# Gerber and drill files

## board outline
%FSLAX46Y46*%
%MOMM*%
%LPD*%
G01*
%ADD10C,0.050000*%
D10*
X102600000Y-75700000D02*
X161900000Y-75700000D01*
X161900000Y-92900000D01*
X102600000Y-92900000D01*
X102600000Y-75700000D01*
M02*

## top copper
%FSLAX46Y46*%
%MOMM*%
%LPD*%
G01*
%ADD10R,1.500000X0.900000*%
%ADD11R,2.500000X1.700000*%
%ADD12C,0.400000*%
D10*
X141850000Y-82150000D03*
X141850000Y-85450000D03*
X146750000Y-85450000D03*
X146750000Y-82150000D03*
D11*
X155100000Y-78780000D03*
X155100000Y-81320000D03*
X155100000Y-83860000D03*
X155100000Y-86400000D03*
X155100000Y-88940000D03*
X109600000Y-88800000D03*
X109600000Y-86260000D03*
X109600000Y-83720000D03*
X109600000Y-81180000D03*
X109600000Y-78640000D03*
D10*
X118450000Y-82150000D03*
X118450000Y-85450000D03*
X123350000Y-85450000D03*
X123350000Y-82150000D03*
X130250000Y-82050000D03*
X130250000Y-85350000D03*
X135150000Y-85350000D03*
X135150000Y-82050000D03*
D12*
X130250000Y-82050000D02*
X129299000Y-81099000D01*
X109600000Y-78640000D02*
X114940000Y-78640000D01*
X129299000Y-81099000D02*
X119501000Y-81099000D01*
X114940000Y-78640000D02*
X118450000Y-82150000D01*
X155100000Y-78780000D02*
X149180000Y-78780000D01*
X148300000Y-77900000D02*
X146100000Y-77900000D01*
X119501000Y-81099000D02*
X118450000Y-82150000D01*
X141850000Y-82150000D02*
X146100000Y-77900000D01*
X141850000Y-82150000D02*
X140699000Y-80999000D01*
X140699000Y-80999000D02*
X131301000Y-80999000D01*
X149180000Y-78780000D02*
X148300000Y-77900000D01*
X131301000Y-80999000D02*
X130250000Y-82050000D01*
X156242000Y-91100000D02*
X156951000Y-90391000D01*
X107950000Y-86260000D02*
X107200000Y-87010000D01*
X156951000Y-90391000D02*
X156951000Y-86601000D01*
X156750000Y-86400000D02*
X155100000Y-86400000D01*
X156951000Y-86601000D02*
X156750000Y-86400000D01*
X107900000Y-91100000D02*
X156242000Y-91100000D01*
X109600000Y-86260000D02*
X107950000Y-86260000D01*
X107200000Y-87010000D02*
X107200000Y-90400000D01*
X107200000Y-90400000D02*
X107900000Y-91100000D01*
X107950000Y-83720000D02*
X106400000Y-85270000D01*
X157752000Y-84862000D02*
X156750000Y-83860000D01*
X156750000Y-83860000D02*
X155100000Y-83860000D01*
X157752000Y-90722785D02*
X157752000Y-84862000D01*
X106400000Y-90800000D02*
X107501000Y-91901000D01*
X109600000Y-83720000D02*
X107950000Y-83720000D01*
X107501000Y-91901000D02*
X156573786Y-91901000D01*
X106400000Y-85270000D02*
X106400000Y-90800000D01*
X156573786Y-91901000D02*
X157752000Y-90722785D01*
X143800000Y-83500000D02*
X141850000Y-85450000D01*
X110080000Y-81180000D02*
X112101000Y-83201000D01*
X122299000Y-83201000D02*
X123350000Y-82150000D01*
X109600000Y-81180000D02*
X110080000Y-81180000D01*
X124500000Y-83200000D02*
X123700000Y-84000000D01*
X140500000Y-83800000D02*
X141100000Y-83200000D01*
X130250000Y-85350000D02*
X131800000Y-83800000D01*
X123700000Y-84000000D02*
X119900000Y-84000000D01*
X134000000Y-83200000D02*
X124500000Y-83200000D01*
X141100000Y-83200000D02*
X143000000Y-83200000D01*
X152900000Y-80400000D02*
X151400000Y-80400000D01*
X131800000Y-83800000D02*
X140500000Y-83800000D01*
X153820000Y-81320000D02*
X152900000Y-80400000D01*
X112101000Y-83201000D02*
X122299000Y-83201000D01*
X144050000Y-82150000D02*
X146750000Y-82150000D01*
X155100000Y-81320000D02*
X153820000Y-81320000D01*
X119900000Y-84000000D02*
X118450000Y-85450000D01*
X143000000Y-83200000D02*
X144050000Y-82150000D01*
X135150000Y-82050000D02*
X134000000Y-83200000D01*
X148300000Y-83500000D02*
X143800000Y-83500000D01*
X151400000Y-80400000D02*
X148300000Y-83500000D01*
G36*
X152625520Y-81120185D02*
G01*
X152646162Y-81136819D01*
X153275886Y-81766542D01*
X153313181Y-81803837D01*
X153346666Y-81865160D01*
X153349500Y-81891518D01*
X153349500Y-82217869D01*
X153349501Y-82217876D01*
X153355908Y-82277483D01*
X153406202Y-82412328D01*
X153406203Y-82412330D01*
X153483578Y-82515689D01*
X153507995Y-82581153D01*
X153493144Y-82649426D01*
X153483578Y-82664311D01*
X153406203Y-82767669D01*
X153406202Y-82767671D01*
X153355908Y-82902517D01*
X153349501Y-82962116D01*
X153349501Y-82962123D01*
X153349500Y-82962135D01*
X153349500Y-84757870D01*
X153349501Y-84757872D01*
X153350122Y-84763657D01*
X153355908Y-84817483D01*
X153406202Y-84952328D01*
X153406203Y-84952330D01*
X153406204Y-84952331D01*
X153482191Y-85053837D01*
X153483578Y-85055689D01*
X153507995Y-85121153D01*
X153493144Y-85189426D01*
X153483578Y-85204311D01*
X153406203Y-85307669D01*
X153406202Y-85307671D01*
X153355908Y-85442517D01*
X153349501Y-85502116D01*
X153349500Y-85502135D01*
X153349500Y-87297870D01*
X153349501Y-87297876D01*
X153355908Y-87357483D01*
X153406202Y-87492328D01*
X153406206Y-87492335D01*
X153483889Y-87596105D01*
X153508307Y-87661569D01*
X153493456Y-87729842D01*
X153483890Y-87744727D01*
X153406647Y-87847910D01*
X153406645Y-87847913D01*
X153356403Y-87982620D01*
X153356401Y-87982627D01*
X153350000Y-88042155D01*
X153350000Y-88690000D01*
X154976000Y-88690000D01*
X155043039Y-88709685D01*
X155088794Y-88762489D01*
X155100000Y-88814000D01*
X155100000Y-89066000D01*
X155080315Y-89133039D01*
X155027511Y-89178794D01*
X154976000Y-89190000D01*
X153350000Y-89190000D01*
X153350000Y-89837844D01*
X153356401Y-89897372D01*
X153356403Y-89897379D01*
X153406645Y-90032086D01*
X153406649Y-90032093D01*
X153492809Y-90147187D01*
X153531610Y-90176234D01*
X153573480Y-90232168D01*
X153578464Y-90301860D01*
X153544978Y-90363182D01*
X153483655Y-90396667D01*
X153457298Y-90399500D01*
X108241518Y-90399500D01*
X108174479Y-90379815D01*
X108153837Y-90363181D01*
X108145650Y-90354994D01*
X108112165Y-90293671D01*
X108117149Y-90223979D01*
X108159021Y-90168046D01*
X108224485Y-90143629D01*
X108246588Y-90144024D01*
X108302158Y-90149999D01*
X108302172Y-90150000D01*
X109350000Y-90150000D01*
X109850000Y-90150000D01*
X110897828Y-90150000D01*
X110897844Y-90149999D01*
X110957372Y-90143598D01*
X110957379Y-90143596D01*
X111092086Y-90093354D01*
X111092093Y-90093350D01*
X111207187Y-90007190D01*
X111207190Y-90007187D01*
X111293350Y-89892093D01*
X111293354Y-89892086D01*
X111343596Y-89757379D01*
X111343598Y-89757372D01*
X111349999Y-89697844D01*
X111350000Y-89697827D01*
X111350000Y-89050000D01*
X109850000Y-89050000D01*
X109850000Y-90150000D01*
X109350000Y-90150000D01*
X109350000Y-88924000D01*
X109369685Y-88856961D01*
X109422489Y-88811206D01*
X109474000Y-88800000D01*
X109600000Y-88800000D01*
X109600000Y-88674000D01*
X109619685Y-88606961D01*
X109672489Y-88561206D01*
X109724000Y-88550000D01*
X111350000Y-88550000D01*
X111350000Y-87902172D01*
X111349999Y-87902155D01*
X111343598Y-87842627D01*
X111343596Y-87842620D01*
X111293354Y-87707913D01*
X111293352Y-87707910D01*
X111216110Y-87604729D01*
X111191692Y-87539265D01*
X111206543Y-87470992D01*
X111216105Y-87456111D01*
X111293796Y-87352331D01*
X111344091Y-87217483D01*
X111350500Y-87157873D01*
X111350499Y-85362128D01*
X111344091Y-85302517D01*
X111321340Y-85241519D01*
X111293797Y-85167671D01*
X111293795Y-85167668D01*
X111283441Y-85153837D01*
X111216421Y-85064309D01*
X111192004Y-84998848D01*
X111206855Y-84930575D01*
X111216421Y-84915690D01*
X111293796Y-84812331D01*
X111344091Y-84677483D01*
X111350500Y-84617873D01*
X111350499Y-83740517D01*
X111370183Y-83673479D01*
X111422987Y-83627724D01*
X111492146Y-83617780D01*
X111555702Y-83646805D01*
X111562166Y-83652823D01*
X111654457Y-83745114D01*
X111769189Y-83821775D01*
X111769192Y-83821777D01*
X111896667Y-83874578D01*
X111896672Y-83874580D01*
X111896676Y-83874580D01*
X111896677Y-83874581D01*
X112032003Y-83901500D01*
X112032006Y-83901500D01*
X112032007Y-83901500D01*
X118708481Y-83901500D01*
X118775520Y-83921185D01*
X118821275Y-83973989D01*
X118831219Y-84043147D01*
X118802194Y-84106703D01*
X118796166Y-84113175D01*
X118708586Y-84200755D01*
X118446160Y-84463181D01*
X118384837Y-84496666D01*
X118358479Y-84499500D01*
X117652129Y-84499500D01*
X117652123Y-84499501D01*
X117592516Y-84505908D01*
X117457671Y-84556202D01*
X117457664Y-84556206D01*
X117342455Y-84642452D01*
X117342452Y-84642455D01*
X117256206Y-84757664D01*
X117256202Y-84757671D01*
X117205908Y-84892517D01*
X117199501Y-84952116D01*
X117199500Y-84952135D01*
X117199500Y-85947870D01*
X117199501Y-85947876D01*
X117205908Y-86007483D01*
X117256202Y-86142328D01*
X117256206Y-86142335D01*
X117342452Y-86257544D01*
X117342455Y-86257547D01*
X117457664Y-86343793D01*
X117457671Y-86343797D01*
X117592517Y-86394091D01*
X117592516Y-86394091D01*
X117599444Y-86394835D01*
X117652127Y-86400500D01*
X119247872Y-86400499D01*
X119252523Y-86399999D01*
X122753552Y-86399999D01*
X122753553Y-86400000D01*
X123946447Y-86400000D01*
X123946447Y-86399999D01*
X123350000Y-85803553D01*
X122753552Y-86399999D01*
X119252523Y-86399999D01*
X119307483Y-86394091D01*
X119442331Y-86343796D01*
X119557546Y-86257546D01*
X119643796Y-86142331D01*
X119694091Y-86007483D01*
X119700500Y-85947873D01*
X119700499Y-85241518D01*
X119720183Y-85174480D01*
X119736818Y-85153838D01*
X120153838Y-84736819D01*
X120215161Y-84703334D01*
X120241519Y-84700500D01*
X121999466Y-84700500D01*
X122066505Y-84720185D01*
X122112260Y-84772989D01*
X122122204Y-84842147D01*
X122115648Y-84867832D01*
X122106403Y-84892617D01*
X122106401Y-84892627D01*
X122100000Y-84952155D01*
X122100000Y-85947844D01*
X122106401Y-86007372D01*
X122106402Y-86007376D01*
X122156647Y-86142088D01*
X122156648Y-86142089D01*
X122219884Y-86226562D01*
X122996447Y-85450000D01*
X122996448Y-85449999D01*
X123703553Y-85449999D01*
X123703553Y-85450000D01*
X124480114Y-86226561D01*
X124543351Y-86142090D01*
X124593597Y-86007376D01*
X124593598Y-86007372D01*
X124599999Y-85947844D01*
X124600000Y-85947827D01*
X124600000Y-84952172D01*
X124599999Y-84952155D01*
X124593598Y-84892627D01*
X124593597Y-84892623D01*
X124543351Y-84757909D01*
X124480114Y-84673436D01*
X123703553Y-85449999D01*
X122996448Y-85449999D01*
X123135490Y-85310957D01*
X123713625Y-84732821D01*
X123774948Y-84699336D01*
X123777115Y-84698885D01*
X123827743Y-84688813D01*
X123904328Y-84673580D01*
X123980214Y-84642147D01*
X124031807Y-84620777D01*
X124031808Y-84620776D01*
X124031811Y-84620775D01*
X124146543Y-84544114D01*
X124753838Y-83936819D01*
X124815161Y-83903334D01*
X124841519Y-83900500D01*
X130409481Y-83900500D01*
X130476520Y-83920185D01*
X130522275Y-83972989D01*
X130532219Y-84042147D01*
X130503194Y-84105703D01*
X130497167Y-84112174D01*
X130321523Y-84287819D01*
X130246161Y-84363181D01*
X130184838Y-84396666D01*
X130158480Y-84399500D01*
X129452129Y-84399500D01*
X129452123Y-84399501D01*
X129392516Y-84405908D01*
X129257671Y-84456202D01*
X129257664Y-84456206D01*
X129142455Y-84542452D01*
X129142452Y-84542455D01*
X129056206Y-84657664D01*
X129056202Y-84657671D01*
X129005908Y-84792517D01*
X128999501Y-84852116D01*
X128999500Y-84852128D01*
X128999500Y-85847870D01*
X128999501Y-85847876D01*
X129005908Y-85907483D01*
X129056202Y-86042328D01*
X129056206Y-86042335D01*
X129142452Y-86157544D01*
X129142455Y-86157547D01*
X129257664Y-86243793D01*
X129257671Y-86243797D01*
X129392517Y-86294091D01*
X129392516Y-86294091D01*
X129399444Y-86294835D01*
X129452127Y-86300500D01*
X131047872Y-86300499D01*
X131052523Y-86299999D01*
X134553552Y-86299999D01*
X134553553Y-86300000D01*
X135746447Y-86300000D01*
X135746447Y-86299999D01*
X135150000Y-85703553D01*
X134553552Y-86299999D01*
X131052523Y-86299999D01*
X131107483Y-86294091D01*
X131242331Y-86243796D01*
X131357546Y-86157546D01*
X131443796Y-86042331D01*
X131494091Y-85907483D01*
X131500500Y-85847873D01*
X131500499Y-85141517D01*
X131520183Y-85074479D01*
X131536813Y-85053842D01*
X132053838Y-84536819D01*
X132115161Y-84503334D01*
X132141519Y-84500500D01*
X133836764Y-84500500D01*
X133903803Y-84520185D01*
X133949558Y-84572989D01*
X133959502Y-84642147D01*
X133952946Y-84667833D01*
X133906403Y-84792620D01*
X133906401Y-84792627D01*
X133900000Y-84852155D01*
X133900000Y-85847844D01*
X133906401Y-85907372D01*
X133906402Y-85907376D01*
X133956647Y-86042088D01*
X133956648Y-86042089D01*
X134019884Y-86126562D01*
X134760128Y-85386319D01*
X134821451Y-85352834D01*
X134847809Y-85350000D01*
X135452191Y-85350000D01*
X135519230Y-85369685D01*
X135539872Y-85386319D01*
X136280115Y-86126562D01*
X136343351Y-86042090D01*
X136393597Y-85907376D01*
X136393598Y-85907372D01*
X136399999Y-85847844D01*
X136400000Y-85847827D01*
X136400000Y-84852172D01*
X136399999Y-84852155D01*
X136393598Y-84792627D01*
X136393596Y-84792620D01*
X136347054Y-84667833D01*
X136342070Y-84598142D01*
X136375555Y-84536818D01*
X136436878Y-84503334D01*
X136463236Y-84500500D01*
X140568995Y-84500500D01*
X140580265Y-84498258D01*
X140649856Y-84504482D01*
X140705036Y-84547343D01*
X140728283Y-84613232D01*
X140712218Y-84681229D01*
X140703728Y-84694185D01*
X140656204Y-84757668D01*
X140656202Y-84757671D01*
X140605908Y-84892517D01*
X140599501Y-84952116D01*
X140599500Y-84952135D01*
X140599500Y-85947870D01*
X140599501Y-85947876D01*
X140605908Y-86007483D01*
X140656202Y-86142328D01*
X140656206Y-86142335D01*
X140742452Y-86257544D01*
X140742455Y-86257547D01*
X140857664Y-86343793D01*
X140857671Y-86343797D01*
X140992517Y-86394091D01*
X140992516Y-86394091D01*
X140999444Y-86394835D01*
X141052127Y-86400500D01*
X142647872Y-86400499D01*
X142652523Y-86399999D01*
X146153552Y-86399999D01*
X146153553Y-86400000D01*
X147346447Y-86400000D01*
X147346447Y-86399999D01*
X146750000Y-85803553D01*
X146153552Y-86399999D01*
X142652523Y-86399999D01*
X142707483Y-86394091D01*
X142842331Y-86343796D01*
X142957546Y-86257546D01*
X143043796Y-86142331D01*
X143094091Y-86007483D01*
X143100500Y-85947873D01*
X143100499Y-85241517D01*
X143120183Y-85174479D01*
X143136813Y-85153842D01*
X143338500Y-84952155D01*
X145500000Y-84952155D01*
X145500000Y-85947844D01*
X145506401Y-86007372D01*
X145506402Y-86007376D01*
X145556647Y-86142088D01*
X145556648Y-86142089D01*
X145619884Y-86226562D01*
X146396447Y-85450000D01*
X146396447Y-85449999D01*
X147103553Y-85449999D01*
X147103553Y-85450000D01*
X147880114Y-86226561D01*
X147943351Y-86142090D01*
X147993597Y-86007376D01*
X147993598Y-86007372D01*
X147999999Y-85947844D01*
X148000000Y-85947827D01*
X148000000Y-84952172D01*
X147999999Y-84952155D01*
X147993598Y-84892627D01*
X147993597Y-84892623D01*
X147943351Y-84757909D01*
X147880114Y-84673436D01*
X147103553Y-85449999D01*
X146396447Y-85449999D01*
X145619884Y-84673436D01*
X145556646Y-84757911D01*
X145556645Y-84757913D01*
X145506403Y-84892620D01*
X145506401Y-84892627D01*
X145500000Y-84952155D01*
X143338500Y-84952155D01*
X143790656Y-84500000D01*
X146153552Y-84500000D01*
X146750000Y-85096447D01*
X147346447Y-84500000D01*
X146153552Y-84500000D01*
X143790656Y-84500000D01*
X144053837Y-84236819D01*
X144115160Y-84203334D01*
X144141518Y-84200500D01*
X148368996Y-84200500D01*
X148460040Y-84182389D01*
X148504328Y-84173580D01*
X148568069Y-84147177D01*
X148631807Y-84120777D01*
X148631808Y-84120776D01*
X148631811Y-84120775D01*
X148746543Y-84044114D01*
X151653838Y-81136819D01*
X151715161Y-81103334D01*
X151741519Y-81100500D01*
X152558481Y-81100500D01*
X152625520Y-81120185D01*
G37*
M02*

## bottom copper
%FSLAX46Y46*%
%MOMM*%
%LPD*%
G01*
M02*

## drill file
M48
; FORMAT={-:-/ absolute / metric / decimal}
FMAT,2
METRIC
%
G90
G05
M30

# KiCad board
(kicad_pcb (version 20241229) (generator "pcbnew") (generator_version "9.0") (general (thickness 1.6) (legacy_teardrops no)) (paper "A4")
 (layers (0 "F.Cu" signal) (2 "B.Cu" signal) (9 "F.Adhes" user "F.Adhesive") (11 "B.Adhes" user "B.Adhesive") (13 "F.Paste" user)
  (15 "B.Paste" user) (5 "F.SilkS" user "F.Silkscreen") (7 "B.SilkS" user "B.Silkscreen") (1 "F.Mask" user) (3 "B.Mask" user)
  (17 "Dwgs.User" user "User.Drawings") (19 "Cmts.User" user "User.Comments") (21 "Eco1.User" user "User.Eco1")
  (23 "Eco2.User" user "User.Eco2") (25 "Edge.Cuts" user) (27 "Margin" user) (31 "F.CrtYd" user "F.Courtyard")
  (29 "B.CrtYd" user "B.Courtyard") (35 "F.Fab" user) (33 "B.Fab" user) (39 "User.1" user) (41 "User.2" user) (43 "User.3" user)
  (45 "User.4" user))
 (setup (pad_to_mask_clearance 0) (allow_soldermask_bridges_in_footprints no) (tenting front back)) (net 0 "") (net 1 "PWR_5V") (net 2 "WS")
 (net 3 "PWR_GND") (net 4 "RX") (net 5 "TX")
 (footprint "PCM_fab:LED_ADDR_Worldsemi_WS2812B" (layer "F.Cu") (at 144.3 83.8)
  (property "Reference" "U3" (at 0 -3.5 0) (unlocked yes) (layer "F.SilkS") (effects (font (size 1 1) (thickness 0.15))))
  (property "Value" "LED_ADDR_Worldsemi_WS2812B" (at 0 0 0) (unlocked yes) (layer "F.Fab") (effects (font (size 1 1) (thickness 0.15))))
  (pad "1" smd rect (at -2.45 -1.65) (size 1.5 0.9) (layers "F.Cu" "F.Mask" "F.Paste") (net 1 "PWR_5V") (thermal_bridge_angle 45))
  (pad "2" smd rect (at -2.45 1.65) (size 1.5 0.9) (layers "F.Cu" "F.Mask" "F.Paste") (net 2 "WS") (thermal_bridge_angle 45))
  (pad "3" smd rect (at 2.45 1.65) (size 1.5 0.9) (layers "F.Cu" "F.Mask" "F.Paste") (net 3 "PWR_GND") (thermal_bridge_angle 45))
  (pad "4" smd rect (at 2.45 -1.65) (size 1.5 0.9) (layers "F.Cu" "F.Mask" "F.Paste") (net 2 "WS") (thermal_bridge_angle 45)))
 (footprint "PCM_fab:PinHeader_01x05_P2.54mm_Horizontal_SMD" (layer "F.Cu") (at 155.1 78.78)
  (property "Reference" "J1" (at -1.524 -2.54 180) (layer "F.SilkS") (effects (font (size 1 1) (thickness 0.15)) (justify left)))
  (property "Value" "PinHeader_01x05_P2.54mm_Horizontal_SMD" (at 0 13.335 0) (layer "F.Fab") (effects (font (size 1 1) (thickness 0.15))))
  (pad "1" smd rect (at 0 0) (size 2.5 1.7) (layers "F.Cu" "F.Mask" "F.Paste") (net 1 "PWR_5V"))
  (pad "2" smd rect (at 0 2.54) (size 2.5 1.7) (layers "F.Cu" "F.Mask" "F.Paste") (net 2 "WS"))
  (pad "3" smd rect (at 0 5.08) (size 2.5 1.7) (layers "F.Cu" "F.Mask" "F.Paste") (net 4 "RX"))
  (pad "4" smd rect (at 0 7.62) (size 2.5 1.7) (layers "F.Cu" "F.Mask" "F.Paste") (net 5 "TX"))
  (pad "5" smd rect (at 0 10.16) (size 2.5 1.7) (layers "F.Cu" "F.Mask" "F.Paste") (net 3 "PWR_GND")))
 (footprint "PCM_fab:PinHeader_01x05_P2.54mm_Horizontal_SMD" (layer "F.Cu") (at 109.6 88.8 180)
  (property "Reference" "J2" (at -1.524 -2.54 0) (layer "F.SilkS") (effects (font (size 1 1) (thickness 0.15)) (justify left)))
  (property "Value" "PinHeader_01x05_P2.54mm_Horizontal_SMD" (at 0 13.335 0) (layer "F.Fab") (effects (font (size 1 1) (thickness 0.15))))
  (pad "1" smd rect (at 0 0 180) (size 2.5 1.7) (layers "F.Cu" "F.Mask" "F.Paste") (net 3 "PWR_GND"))
  (pad "2" smd rect (at 0 2.54 180) (size 2.5 1.7) (layers "F.Cu" "F.Mask" "F.Paste") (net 5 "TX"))
  (pad "3" smd rect (at 0 5.08 180) (size 2.5 1.7) (layers "F.Cu" "F.Mask" "F.Paste") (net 4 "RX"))
  (pad "4" smd rect (at 0 7.62 180) (size 2.5 1.7) (layers "F.Cu" "F.Mask" "F.Paste") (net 2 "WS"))
  (pad "5" smd rect (at 0 10.16 180) (size 2.5 1.7) (layers "F.Cu" "F.Mask" "F.Paste") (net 1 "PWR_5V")))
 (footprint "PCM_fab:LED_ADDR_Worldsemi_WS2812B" (layer "F.Cu") (at 120.9 83.8)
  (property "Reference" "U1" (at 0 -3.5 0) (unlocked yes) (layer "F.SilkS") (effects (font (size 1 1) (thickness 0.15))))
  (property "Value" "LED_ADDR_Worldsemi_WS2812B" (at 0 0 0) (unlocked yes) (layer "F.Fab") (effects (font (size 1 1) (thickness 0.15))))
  (pad "1" smd rect (at -2.45 -1.65) (size 1.5 0.9) (layers "F.Cu" "F.Mask" "F.Paste") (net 1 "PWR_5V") (thermal_bridge_angle 45))
  (pad "2" smd rect (at -2.45 1.65) (size 1.5 0.9) (layers "F.Cu" "F.Mask" "F.Paste") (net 2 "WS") (thermal_bridge_angle 45))
  (pad "3" smd rect (at 2.45 1.65) (size 1.5 0.9) (layers "F.Cu" "F.Mask" "F.Paste") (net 3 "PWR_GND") (thermal_bridge_angle 45))
  (pad "4" smd rect (at 2.45 -1.65) (size 1.5 0.9) (layers "F.Cu" "F.Mask" "F.Paste") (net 2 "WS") (thermal_bridge_angle 45)))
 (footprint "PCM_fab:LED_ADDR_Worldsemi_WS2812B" (layer "F.Cu") (at 132.7 83.7)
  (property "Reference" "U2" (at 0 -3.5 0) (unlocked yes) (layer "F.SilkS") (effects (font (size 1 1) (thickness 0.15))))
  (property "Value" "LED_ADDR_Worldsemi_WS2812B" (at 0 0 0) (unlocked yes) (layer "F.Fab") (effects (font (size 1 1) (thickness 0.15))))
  (pad "1" smd rect (at -2.45 -1.65) (size 1.5 0.9) (layers "F.Cu" "F.Mask" "F.Paste") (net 1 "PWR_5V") (thermal_bridge_angle 45))
  (pad "2" smd rect (at -2.45 1.65) (size 1.5 0.9) (layers "F.Cu" "F.Mask" "F.Paste") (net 2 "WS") (thermal_bridge_angle 45))
  (pad "3" smd rect (at 2.45 1.65) (size 1.5 0.9) (layers "F.Cu" "F.Mask" "F.Paste") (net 3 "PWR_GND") (thermal_bridge_angle 45))
  (pad "4" smd rect (at 2.45 -1.65) (size 1.5 0.9) (layers "F.Cu" "F.Mask" "F.Paste") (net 2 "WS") (thermal_bridge_angle 45)))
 (gr_rect (start 102.6 75.7) (end 161.9 92.9) (stroke (width 0.05) (type default)) (fill no) (layer "Edge.Cuts"))
 (segment (start 130.25 82.05) (end 129.299 81.099) (width 0.4) (layer "F.Cu") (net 1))
 (segment (start 109.6 78.64) (end 114.94 78.64) (width 0.4) (layer "F.Cu") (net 1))
 (segment (start 129.299 81.099) (end 119.501 81.099) (width 0.4) (layer "F.Cu") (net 1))
 (segment (start 114.94 78.64) (end 118.45 82.15) (width 0.4) (layer "F.Cu") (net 1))
 (segment (start 155.1 78.78) (end 149.18 78.78) (width 0.4) (layer "F.Cu") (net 1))
 (segment (start 148.3 77.9) (end 146.1 77.9) (width 0.4) (layer "F.Cu") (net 1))
 (segment (start 119.501 81.099) (end 118.45 82.15) (width 0.4) (layer "F.Cu") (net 1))
 (segment (start 141.85 82.15) (end 146.1 77.9) (width 0.4) (layer "F.Cu") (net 1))
 (segment (start 141.85 82.15) (end 140.699 80.999) (width 0.4) (layer "F.Cu") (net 1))
 (segment (start 140.699 80.999) (end 131.301 80.999) (width 0.4) (layer "F.Cu") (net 1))
 (segment (start 149.18 78.78) (end 148.3 77.9) (width 0.4) (layer "F.Cu") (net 1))
 (segment (start 131.301 80.999) (end 130.25 82.05) (width 0.4) (layer "F.Cu") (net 1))
 (segment (start 156.242 91.1) (end 156.951 90.391) (width 0.4) (layer "F.Cu") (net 5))
 (segment (start 107.95 86.26) (end 107.2 87.01) (width 0.4) (layer "F.Cu") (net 5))
 (segment (start 156.951 90.391) (end 156.951 86.601) (width 0.4) (layer "F.Cu") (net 5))
 (segment (start 156.75 86.4) (end 155.1 86.4) (width 0.4) (layer "F.Cu") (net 5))
 (segment (start 156.951 86.601) (end 156.75 86.4) (width 0.4) (layer "F.Cu") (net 5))
 (segment (start 107.9 91.1) (end 156.242 91.1) (width 0.4) (layer "F.Cu") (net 5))
 (segment (start 109.6 86.26) (end 107.95 86.26) (width 0.4) (layer "F.Cu") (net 5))
 (segment (start 107.2 87.01) (end 107.2 90.4) (width 0.4) (layer "F.Cu") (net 5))
 (segment (start 107.2 90.4) (end 107.9 91.1) (width 0.4) (layer "F.Cu") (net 5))
 (segment (start 107.95 83.72) (end 106.4 85.27) (width 0.4) (layer "F.Cu") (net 4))
 (segment (start 157.752 84.862) (end 156.75 83.86) (width 0.4) (layer "F.Cu") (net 4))
 (segment (start 156.75 83.86) (end 155.1 83.86) (width 0.4) (layer "F.Cu") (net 4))
 (segment (start 157.752 90.722785) (end 157.752 84.862) (width 0.4) (layer "F.Cu") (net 4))
 (segment (start 106.4 90.8) (end 107.501 91.901) (width 0.4) (layer "F.Cu") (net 4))
 (segment (start 109.6 83.72) (end 107.95 83.72) (width 0.4) (layer "F.Cu") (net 4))
 (segment (start 107.501 91.901) (end 156.573786 91.901) (width 0.4) (layer "F.Cu") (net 4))
 (segment (start 106.4 85.27) (end 106.4 90.8) (width 0.4) (layer "F.Cu") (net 4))
 (segment (start 156.573786 91.901) (end 157.752 90.722785) (width 0.4) (layer "F.Cu") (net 4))
 (segment (start 143.8 83.5) (end 141.85 85.45) (width 0.4) (layer "F.Cu") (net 2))
 (segment (start 110.08 81.18) (end 112.101 83.201) (width 0.4) (layer "F.Cu") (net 2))
 (segment (start 122.299 83.201) (end 123.35 82.15) (width 0.4) (layer "F.Cu") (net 2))
 (segment (start 109.6 81.18) (end 110.08 81.18) (width 0.4) (layer "F.Cu") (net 2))
 (segment (start 124.5 83.2) (end 123.7 84) (width 0.4) (layer "F.Cu") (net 2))
 (segment (start 140.5 83.8) (end 141.1 83.2) (width 0.4) (layer "F.Cu") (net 2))
 (segment (start 130.25 85.35) (end 131.8 83.8) (width 0.4) (layer "F.Cu") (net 2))
 (segment (start 123.7 84) (end 119.9 84) (width 0.4) (layer "F.Cu") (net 2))
 (segment (start 134 83.2) (end 124.5 83.2) (width 0.4) (layer "F.Cu") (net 2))
 (segment (start 141.1 83.2) (end 143 83.2) (width 0.4) (layer "F.Cu") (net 2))
 (segment (start 152.9 80.4) (end 151.4 80.4) (width 0.4) (layer "F.Cu") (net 2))
 (segment (start 131.8 83.8) (end 140.5 83.8) (width 0.4) (layer "F.Cu") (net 2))
 (segment (start 153.82 81.32) (end 152.9 80.4) (width 0.4) (layer "F.Cu") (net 2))
 (segment (start 112.101 83.201) (end 122.299 83.201) (width 0.4) (layer "F.Cu") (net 2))
 (segment (start 144.05 82.15) (end 146.75 82.15) (width 0.4) (layer "F.Cu") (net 2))
 (segment (start 155.1 81.32) (end 153.82 81.32) (width 0.4) (layer "F.Cu") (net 2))
 (segment (start 119.9 84) (end 118.45 85.45) (width 0.4) (layer "F.Cu") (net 2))
 (segment (start 143 83.2) (end 144.05 82.15) (width 0.4) (layer "F.Cu") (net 2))
 (segment (start 135.15 82.05) (end 134 83.2) (width 0.4) (layer "F.Cu") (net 2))
 (segment (start 148.3 83.5) (end 143.8 83.5) (width 0.4) (layer "F.Cu") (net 2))
 (segment (start 151.4 80.4) (end 148.3 83.5) (width 0.4) (layer "F.Cu") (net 2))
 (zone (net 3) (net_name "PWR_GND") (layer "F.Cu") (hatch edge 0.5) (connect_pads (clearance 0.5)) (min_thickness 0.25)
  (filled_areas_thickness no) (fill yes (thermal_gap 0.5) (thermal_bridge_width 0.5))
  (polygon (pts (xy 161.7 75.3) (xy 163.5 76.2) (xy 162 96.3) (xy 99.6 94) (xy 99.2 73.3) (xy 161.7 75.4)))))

